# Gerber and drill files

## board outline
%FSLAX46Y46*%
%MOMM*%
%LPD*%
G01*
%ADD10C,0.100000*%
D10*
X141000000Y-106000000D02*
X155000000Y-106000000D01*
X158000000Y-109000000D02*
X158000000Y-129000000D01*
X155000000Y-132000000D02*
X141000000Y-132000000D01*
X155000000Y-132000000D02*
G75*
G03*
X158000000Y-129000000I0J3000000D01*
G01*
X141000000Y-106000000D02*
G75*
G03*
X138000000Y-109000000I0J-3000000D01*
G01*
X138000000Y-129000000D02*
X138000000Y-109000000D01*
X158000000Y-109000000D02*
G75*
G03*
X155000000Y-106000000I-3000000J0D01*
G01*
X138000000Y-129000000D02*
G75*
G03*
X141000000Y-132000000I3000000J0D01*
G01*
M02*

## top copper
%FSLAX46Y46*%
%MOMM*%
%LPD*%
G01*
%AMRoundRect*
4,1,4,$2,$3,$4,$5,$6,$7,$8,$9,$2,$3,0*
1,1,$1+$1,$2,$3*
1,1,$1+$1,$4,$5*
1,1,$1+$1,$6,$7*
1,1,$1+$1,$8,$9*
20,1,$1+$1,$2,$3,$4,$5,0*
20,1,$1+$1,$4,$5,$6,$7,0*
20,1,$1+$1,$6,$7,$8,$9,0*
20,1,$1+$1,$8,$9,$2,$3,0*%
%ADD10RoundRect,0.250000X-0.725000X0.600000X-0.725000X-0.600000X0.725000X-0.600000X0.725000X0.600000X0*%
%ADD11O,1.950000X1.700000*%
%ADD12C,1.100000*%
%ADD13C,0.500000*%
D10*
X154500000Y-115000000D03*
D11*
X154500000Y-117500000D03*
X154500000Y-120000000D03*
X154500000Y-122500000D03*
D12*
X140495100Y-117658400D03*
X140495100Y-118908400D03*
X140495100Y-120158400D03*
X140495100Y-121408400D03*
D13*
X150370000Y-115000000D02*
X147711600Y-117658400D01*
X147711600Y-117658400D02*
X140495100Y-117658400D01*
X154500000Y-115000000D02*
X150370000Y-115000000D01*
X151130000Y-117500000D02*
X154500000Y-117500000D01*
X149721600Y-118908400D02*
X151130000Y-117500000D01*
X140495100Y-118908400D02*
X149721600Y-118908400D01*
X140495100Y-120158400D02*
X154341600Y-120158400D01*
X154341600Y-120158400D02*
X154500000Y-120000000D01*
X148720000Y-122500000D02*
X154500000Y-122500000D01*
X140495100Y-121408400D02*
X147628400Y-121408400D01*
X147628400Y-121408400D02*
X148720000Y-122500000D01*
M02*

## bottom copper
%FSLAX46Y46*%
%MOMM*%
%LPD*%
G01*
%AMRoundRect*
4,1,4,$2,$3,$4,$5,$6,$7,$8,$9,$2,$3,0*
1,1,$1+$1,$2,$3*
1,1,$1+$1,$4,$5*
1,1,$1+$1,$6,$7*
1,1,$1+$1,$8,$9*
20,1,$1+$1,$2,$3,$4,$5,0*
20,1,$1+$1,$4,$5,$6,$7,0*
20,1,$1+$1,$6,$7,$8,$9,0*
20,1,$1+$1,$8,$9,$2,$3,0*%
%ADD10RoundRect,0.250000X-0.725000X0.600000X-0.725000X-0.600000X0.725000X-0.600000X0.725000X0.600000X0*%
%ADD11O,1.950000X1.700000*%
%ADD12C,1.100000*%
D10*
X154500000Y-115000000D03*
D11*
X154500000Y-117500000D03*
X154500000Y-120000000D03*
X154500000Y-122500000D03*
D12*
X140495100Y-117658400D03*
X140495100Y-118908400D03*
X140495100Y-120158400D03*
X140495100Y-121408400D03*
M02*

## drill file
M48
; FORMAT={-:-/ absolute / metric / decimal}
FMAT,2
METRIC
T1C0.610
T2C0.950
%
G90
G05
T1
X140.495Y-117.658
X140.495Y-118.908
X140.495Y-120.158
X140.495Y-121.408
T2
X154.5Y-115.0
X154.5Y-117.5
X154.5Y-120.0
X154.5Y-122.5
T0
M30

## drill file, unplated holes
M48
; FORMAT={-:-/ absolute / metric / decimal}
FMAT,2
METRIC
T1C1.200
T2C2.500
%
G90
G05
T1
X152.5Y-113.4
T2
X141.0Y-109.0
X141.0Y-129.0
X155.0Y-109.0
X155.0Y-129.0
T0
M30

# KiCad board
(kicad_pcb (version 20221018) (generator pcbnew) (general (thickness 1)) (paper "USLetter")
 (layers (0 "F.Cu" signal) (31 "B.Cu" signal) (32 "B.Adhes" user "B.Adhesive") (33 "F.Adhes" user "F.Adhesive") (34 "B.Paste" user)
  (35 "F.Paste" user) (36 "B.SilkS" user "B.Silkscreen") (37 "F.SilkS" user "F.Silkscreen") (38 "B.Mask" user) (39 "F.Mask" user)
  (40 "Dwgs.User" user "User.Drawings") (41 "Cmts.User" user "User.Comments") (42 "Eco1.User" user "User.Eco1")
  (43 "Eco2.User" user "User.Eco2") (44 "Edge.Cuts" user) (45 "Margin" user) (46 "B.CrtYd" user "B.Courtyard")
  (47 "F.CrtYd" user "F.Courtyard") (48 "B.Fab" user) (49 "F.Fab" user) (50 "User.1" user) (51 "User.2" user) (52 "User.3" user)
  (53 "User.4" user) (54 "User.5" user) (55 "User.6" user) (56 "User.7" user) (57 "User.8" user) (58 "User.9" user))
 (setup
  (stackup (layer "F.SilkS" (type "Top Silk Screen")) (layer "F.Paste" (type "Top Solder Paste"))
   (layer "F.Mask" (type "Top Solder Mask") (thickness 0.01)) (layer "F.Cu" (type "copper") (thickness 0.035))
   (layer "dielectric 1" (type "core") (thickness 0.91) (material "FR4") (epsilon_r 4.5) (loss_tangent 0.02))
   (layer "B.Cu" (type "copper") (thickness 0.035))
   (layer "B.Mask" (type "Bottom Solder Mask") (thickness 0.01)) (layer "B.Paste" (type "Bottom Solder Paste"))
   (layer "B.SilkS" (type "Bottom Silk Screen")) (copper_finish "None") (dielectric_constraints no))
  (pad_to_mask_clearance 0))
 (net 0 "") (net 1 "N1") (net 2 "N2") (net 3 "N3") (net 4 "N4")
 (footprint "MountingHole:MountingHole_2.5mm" (layer "F.Cu") (at 141 109)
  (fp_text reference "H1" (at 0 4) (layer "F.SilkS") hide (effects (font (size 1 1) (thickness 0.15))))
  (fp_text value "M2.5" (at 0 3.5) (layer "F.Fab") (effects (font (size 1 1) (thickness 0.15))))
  (pad "" np_thru_hole circle (at 0 0) (size 2.5 2.5) (drill 2.5) (layers "*.Cu" "*.Mask")))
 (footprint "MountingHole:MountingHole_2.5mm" (layer "F.Cu") (at 155 109)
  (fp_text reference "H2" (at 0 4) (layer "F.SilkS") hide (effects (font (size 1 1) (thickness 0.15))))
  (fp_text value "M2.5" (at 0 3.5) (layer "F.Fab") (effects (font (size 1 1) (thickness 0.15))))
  (pad "" np_thru_hole circle (at 0 0) (size 2.5 2.5) (drill 2.5) (layers "*.Cu" "*.Mask")))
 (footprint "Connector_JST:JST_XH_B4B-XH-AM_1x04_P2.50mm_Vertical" (layer "F.Cu") (at 154.5 115 -90)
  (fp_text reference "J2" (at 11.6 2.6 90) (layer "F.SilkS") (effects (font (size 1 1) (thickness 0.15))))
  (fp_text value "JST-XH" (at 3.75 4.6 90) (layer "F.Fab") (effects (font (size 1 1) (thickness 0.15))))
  (pad "" np_thru_hole circle (at -1.6 2 270) (size 1.2 1.2) (drill 1.2) (layers "*.Cu" "*.Mask"))
  (pad "1" thru_hole roundrect (at 0 0 270) (size 1.7 1.95) (drill 0.95) (layers "*.Cu" "*.Mask") (roundrect_rratio 0.1470588235)
   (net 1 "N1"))
  (pad "2" thru_hole oval (at 2.5 0 270) (size 1.7 1.95) (drill 0.95) (layers "*.Cu" "*.Mask") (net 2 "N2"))
  (pad "3" thru_hole oval (at 5 0 270) (size 1.7 1.95) (drill 0.95) (layers "*.Cu" "*.Mask") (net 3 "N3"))
  (pad "4" thru_hole oval (at 7.5 0 270) (size 1.7 1.95) (drill 0.95) (layers "*.Cu" "*.Mask") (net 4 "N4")))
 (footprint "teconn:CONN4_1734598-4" (layer "F.Cu") (at 140.4951 117.6584 90)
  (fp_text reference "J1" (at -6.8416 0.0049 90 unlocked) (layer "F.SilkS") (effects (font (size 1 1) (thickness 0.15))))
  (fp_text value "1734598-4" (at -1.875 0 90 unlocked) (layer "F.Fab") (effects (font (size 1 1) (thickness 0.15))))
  (pad "1" thru_hole circle (at 0 0 90) (size 1.1 1.1) (drill 0.6096) (layers "*.Cu" "*.Mask") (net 1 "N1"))
  (pad "2" thru_hole circle (at -1.25 0 90) (size 1.1 1.1) (drill 0.6096) (layers "*.Cu" "*.Mask") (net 2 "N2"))
  (pad "3" thru_hole circle (at -2.5 0 90) (size 1.1 1.1) (drill 0.6096) (layers "*.Cu" "*.Mask") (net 3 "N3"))
  (pad "4" thru_hole circle (at -3.75 0 90) (size 1.1 1.1) (drill 0.6096) (layers "*.Cu" "*.Mask") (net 4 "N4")))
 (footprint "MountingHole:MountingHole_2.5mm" (layer "F.Cu") (at 141 129)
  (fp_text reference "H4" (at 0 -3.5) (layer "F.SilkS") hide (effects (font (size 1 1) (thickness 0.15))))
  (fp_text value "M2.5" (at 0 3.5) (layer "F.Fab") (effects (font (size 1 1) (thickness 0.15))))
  (pad "" np_thru_hole circle (at 0 0) (size 2.5 2.5) (drill 2.5) (layers "*.Cu" "*.Mask")))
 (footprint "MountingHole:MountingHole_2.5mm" (layer "F.Cu") (at 155 129)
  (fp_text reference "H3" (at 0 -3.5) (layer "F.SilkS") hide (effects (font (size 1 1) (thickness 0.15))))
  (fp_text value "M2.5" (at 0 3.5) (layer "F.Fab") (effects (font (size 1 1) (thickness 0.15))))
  (pad "" np_thru_hole circle (at 0 0) (size 2.5 2.5) (drill 2.5) (layers "*.Cu" "*.Mask")))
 (gr_line (start 141 106) (end 155 106) (stroke (width 0.1) (type default)) (layer "Edge.Cuts"))
 (gr_line (start 158 109) (end 158 129) (stroke (width 0.1) (type default)) (layer "Edge.Cuts"))
 (gr_line (start 155 132) (end 141 132) (stroke (width 0.1) (type default)) (layer "Edge.Cuts"))
 (gr_arc (start 158 129) (mid 157.12132 131.12132) (end 155 132) (stroke (width 0.1) (type default)) (layer "Edge.Cuts"))
 (gr_arc (start 138 109) (mid 138.87868 106.87868) (end 141 106) (stroke (width 0.1) (type default)) (layer "Edge.Cuts"))
 (gr_line (start 138 129) (end 138 109) (stroke (width 0.1) (type default)) (layer "Edge.Cuts"))
 (gr_arc (start 155 106) (mid 157.12132 106.87868) (end 158 109) (stroke (width 0.1) (type default)) (layer "Edge.Cuts"))
 (gr_arc (start 141 132) (mid 138.87868 131.12132) (end 138 129) (stroke (width 0.1) (type default)) (layer "Edge.Cuts"))
 (segment (start 150.37 115) (end 147.7116 117.6584) (width 0.5) (layer "F.Cu") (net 1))
 (segment (start 147.7116 117.6584) (end 140.4951 117.6584) (width 0.5) (layer "F.Cu") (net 1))
 (segment (start 154.5 115) (end 150.37 115) (width 0.5) (layer "F.Cu") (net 1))
 (segment (start 151.13 117.5) (end 154.5 117.5) (width 0.5) (layer "F.Cu") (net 2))
 (segment (start 149.7216 118.9084) (end 151.13 117.5) (width 0.5) (layer "F.Cu") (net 2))
 (segment (start 140.4951 118.9084) (end 149.7216 118.9084) (width 0.5) (layer "F.Cu") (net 2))
 (segment (start 140.4951 120.1584) (end 154.3416 120.1584) (width 0.5) (layer "F.Cu") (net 3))
 (segment (start 154.3416 120.1584) (end 154.5 120) (width 0.5) (layer "F.Cu") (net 3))
 (segment (start 148.72 122.5) (end 154.5 122.5) (width 0.5) (layer "F.Cu") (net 4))
 (segment (start 140.4951 121.4084) (end 147.6284 121.4084) (width 0.5) (layer "F.Cu") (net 4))
 (segment (start 147.6284 121.4084) (end 148.72 122.5) (width 0.5) (layer "F.Cu") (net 4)))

